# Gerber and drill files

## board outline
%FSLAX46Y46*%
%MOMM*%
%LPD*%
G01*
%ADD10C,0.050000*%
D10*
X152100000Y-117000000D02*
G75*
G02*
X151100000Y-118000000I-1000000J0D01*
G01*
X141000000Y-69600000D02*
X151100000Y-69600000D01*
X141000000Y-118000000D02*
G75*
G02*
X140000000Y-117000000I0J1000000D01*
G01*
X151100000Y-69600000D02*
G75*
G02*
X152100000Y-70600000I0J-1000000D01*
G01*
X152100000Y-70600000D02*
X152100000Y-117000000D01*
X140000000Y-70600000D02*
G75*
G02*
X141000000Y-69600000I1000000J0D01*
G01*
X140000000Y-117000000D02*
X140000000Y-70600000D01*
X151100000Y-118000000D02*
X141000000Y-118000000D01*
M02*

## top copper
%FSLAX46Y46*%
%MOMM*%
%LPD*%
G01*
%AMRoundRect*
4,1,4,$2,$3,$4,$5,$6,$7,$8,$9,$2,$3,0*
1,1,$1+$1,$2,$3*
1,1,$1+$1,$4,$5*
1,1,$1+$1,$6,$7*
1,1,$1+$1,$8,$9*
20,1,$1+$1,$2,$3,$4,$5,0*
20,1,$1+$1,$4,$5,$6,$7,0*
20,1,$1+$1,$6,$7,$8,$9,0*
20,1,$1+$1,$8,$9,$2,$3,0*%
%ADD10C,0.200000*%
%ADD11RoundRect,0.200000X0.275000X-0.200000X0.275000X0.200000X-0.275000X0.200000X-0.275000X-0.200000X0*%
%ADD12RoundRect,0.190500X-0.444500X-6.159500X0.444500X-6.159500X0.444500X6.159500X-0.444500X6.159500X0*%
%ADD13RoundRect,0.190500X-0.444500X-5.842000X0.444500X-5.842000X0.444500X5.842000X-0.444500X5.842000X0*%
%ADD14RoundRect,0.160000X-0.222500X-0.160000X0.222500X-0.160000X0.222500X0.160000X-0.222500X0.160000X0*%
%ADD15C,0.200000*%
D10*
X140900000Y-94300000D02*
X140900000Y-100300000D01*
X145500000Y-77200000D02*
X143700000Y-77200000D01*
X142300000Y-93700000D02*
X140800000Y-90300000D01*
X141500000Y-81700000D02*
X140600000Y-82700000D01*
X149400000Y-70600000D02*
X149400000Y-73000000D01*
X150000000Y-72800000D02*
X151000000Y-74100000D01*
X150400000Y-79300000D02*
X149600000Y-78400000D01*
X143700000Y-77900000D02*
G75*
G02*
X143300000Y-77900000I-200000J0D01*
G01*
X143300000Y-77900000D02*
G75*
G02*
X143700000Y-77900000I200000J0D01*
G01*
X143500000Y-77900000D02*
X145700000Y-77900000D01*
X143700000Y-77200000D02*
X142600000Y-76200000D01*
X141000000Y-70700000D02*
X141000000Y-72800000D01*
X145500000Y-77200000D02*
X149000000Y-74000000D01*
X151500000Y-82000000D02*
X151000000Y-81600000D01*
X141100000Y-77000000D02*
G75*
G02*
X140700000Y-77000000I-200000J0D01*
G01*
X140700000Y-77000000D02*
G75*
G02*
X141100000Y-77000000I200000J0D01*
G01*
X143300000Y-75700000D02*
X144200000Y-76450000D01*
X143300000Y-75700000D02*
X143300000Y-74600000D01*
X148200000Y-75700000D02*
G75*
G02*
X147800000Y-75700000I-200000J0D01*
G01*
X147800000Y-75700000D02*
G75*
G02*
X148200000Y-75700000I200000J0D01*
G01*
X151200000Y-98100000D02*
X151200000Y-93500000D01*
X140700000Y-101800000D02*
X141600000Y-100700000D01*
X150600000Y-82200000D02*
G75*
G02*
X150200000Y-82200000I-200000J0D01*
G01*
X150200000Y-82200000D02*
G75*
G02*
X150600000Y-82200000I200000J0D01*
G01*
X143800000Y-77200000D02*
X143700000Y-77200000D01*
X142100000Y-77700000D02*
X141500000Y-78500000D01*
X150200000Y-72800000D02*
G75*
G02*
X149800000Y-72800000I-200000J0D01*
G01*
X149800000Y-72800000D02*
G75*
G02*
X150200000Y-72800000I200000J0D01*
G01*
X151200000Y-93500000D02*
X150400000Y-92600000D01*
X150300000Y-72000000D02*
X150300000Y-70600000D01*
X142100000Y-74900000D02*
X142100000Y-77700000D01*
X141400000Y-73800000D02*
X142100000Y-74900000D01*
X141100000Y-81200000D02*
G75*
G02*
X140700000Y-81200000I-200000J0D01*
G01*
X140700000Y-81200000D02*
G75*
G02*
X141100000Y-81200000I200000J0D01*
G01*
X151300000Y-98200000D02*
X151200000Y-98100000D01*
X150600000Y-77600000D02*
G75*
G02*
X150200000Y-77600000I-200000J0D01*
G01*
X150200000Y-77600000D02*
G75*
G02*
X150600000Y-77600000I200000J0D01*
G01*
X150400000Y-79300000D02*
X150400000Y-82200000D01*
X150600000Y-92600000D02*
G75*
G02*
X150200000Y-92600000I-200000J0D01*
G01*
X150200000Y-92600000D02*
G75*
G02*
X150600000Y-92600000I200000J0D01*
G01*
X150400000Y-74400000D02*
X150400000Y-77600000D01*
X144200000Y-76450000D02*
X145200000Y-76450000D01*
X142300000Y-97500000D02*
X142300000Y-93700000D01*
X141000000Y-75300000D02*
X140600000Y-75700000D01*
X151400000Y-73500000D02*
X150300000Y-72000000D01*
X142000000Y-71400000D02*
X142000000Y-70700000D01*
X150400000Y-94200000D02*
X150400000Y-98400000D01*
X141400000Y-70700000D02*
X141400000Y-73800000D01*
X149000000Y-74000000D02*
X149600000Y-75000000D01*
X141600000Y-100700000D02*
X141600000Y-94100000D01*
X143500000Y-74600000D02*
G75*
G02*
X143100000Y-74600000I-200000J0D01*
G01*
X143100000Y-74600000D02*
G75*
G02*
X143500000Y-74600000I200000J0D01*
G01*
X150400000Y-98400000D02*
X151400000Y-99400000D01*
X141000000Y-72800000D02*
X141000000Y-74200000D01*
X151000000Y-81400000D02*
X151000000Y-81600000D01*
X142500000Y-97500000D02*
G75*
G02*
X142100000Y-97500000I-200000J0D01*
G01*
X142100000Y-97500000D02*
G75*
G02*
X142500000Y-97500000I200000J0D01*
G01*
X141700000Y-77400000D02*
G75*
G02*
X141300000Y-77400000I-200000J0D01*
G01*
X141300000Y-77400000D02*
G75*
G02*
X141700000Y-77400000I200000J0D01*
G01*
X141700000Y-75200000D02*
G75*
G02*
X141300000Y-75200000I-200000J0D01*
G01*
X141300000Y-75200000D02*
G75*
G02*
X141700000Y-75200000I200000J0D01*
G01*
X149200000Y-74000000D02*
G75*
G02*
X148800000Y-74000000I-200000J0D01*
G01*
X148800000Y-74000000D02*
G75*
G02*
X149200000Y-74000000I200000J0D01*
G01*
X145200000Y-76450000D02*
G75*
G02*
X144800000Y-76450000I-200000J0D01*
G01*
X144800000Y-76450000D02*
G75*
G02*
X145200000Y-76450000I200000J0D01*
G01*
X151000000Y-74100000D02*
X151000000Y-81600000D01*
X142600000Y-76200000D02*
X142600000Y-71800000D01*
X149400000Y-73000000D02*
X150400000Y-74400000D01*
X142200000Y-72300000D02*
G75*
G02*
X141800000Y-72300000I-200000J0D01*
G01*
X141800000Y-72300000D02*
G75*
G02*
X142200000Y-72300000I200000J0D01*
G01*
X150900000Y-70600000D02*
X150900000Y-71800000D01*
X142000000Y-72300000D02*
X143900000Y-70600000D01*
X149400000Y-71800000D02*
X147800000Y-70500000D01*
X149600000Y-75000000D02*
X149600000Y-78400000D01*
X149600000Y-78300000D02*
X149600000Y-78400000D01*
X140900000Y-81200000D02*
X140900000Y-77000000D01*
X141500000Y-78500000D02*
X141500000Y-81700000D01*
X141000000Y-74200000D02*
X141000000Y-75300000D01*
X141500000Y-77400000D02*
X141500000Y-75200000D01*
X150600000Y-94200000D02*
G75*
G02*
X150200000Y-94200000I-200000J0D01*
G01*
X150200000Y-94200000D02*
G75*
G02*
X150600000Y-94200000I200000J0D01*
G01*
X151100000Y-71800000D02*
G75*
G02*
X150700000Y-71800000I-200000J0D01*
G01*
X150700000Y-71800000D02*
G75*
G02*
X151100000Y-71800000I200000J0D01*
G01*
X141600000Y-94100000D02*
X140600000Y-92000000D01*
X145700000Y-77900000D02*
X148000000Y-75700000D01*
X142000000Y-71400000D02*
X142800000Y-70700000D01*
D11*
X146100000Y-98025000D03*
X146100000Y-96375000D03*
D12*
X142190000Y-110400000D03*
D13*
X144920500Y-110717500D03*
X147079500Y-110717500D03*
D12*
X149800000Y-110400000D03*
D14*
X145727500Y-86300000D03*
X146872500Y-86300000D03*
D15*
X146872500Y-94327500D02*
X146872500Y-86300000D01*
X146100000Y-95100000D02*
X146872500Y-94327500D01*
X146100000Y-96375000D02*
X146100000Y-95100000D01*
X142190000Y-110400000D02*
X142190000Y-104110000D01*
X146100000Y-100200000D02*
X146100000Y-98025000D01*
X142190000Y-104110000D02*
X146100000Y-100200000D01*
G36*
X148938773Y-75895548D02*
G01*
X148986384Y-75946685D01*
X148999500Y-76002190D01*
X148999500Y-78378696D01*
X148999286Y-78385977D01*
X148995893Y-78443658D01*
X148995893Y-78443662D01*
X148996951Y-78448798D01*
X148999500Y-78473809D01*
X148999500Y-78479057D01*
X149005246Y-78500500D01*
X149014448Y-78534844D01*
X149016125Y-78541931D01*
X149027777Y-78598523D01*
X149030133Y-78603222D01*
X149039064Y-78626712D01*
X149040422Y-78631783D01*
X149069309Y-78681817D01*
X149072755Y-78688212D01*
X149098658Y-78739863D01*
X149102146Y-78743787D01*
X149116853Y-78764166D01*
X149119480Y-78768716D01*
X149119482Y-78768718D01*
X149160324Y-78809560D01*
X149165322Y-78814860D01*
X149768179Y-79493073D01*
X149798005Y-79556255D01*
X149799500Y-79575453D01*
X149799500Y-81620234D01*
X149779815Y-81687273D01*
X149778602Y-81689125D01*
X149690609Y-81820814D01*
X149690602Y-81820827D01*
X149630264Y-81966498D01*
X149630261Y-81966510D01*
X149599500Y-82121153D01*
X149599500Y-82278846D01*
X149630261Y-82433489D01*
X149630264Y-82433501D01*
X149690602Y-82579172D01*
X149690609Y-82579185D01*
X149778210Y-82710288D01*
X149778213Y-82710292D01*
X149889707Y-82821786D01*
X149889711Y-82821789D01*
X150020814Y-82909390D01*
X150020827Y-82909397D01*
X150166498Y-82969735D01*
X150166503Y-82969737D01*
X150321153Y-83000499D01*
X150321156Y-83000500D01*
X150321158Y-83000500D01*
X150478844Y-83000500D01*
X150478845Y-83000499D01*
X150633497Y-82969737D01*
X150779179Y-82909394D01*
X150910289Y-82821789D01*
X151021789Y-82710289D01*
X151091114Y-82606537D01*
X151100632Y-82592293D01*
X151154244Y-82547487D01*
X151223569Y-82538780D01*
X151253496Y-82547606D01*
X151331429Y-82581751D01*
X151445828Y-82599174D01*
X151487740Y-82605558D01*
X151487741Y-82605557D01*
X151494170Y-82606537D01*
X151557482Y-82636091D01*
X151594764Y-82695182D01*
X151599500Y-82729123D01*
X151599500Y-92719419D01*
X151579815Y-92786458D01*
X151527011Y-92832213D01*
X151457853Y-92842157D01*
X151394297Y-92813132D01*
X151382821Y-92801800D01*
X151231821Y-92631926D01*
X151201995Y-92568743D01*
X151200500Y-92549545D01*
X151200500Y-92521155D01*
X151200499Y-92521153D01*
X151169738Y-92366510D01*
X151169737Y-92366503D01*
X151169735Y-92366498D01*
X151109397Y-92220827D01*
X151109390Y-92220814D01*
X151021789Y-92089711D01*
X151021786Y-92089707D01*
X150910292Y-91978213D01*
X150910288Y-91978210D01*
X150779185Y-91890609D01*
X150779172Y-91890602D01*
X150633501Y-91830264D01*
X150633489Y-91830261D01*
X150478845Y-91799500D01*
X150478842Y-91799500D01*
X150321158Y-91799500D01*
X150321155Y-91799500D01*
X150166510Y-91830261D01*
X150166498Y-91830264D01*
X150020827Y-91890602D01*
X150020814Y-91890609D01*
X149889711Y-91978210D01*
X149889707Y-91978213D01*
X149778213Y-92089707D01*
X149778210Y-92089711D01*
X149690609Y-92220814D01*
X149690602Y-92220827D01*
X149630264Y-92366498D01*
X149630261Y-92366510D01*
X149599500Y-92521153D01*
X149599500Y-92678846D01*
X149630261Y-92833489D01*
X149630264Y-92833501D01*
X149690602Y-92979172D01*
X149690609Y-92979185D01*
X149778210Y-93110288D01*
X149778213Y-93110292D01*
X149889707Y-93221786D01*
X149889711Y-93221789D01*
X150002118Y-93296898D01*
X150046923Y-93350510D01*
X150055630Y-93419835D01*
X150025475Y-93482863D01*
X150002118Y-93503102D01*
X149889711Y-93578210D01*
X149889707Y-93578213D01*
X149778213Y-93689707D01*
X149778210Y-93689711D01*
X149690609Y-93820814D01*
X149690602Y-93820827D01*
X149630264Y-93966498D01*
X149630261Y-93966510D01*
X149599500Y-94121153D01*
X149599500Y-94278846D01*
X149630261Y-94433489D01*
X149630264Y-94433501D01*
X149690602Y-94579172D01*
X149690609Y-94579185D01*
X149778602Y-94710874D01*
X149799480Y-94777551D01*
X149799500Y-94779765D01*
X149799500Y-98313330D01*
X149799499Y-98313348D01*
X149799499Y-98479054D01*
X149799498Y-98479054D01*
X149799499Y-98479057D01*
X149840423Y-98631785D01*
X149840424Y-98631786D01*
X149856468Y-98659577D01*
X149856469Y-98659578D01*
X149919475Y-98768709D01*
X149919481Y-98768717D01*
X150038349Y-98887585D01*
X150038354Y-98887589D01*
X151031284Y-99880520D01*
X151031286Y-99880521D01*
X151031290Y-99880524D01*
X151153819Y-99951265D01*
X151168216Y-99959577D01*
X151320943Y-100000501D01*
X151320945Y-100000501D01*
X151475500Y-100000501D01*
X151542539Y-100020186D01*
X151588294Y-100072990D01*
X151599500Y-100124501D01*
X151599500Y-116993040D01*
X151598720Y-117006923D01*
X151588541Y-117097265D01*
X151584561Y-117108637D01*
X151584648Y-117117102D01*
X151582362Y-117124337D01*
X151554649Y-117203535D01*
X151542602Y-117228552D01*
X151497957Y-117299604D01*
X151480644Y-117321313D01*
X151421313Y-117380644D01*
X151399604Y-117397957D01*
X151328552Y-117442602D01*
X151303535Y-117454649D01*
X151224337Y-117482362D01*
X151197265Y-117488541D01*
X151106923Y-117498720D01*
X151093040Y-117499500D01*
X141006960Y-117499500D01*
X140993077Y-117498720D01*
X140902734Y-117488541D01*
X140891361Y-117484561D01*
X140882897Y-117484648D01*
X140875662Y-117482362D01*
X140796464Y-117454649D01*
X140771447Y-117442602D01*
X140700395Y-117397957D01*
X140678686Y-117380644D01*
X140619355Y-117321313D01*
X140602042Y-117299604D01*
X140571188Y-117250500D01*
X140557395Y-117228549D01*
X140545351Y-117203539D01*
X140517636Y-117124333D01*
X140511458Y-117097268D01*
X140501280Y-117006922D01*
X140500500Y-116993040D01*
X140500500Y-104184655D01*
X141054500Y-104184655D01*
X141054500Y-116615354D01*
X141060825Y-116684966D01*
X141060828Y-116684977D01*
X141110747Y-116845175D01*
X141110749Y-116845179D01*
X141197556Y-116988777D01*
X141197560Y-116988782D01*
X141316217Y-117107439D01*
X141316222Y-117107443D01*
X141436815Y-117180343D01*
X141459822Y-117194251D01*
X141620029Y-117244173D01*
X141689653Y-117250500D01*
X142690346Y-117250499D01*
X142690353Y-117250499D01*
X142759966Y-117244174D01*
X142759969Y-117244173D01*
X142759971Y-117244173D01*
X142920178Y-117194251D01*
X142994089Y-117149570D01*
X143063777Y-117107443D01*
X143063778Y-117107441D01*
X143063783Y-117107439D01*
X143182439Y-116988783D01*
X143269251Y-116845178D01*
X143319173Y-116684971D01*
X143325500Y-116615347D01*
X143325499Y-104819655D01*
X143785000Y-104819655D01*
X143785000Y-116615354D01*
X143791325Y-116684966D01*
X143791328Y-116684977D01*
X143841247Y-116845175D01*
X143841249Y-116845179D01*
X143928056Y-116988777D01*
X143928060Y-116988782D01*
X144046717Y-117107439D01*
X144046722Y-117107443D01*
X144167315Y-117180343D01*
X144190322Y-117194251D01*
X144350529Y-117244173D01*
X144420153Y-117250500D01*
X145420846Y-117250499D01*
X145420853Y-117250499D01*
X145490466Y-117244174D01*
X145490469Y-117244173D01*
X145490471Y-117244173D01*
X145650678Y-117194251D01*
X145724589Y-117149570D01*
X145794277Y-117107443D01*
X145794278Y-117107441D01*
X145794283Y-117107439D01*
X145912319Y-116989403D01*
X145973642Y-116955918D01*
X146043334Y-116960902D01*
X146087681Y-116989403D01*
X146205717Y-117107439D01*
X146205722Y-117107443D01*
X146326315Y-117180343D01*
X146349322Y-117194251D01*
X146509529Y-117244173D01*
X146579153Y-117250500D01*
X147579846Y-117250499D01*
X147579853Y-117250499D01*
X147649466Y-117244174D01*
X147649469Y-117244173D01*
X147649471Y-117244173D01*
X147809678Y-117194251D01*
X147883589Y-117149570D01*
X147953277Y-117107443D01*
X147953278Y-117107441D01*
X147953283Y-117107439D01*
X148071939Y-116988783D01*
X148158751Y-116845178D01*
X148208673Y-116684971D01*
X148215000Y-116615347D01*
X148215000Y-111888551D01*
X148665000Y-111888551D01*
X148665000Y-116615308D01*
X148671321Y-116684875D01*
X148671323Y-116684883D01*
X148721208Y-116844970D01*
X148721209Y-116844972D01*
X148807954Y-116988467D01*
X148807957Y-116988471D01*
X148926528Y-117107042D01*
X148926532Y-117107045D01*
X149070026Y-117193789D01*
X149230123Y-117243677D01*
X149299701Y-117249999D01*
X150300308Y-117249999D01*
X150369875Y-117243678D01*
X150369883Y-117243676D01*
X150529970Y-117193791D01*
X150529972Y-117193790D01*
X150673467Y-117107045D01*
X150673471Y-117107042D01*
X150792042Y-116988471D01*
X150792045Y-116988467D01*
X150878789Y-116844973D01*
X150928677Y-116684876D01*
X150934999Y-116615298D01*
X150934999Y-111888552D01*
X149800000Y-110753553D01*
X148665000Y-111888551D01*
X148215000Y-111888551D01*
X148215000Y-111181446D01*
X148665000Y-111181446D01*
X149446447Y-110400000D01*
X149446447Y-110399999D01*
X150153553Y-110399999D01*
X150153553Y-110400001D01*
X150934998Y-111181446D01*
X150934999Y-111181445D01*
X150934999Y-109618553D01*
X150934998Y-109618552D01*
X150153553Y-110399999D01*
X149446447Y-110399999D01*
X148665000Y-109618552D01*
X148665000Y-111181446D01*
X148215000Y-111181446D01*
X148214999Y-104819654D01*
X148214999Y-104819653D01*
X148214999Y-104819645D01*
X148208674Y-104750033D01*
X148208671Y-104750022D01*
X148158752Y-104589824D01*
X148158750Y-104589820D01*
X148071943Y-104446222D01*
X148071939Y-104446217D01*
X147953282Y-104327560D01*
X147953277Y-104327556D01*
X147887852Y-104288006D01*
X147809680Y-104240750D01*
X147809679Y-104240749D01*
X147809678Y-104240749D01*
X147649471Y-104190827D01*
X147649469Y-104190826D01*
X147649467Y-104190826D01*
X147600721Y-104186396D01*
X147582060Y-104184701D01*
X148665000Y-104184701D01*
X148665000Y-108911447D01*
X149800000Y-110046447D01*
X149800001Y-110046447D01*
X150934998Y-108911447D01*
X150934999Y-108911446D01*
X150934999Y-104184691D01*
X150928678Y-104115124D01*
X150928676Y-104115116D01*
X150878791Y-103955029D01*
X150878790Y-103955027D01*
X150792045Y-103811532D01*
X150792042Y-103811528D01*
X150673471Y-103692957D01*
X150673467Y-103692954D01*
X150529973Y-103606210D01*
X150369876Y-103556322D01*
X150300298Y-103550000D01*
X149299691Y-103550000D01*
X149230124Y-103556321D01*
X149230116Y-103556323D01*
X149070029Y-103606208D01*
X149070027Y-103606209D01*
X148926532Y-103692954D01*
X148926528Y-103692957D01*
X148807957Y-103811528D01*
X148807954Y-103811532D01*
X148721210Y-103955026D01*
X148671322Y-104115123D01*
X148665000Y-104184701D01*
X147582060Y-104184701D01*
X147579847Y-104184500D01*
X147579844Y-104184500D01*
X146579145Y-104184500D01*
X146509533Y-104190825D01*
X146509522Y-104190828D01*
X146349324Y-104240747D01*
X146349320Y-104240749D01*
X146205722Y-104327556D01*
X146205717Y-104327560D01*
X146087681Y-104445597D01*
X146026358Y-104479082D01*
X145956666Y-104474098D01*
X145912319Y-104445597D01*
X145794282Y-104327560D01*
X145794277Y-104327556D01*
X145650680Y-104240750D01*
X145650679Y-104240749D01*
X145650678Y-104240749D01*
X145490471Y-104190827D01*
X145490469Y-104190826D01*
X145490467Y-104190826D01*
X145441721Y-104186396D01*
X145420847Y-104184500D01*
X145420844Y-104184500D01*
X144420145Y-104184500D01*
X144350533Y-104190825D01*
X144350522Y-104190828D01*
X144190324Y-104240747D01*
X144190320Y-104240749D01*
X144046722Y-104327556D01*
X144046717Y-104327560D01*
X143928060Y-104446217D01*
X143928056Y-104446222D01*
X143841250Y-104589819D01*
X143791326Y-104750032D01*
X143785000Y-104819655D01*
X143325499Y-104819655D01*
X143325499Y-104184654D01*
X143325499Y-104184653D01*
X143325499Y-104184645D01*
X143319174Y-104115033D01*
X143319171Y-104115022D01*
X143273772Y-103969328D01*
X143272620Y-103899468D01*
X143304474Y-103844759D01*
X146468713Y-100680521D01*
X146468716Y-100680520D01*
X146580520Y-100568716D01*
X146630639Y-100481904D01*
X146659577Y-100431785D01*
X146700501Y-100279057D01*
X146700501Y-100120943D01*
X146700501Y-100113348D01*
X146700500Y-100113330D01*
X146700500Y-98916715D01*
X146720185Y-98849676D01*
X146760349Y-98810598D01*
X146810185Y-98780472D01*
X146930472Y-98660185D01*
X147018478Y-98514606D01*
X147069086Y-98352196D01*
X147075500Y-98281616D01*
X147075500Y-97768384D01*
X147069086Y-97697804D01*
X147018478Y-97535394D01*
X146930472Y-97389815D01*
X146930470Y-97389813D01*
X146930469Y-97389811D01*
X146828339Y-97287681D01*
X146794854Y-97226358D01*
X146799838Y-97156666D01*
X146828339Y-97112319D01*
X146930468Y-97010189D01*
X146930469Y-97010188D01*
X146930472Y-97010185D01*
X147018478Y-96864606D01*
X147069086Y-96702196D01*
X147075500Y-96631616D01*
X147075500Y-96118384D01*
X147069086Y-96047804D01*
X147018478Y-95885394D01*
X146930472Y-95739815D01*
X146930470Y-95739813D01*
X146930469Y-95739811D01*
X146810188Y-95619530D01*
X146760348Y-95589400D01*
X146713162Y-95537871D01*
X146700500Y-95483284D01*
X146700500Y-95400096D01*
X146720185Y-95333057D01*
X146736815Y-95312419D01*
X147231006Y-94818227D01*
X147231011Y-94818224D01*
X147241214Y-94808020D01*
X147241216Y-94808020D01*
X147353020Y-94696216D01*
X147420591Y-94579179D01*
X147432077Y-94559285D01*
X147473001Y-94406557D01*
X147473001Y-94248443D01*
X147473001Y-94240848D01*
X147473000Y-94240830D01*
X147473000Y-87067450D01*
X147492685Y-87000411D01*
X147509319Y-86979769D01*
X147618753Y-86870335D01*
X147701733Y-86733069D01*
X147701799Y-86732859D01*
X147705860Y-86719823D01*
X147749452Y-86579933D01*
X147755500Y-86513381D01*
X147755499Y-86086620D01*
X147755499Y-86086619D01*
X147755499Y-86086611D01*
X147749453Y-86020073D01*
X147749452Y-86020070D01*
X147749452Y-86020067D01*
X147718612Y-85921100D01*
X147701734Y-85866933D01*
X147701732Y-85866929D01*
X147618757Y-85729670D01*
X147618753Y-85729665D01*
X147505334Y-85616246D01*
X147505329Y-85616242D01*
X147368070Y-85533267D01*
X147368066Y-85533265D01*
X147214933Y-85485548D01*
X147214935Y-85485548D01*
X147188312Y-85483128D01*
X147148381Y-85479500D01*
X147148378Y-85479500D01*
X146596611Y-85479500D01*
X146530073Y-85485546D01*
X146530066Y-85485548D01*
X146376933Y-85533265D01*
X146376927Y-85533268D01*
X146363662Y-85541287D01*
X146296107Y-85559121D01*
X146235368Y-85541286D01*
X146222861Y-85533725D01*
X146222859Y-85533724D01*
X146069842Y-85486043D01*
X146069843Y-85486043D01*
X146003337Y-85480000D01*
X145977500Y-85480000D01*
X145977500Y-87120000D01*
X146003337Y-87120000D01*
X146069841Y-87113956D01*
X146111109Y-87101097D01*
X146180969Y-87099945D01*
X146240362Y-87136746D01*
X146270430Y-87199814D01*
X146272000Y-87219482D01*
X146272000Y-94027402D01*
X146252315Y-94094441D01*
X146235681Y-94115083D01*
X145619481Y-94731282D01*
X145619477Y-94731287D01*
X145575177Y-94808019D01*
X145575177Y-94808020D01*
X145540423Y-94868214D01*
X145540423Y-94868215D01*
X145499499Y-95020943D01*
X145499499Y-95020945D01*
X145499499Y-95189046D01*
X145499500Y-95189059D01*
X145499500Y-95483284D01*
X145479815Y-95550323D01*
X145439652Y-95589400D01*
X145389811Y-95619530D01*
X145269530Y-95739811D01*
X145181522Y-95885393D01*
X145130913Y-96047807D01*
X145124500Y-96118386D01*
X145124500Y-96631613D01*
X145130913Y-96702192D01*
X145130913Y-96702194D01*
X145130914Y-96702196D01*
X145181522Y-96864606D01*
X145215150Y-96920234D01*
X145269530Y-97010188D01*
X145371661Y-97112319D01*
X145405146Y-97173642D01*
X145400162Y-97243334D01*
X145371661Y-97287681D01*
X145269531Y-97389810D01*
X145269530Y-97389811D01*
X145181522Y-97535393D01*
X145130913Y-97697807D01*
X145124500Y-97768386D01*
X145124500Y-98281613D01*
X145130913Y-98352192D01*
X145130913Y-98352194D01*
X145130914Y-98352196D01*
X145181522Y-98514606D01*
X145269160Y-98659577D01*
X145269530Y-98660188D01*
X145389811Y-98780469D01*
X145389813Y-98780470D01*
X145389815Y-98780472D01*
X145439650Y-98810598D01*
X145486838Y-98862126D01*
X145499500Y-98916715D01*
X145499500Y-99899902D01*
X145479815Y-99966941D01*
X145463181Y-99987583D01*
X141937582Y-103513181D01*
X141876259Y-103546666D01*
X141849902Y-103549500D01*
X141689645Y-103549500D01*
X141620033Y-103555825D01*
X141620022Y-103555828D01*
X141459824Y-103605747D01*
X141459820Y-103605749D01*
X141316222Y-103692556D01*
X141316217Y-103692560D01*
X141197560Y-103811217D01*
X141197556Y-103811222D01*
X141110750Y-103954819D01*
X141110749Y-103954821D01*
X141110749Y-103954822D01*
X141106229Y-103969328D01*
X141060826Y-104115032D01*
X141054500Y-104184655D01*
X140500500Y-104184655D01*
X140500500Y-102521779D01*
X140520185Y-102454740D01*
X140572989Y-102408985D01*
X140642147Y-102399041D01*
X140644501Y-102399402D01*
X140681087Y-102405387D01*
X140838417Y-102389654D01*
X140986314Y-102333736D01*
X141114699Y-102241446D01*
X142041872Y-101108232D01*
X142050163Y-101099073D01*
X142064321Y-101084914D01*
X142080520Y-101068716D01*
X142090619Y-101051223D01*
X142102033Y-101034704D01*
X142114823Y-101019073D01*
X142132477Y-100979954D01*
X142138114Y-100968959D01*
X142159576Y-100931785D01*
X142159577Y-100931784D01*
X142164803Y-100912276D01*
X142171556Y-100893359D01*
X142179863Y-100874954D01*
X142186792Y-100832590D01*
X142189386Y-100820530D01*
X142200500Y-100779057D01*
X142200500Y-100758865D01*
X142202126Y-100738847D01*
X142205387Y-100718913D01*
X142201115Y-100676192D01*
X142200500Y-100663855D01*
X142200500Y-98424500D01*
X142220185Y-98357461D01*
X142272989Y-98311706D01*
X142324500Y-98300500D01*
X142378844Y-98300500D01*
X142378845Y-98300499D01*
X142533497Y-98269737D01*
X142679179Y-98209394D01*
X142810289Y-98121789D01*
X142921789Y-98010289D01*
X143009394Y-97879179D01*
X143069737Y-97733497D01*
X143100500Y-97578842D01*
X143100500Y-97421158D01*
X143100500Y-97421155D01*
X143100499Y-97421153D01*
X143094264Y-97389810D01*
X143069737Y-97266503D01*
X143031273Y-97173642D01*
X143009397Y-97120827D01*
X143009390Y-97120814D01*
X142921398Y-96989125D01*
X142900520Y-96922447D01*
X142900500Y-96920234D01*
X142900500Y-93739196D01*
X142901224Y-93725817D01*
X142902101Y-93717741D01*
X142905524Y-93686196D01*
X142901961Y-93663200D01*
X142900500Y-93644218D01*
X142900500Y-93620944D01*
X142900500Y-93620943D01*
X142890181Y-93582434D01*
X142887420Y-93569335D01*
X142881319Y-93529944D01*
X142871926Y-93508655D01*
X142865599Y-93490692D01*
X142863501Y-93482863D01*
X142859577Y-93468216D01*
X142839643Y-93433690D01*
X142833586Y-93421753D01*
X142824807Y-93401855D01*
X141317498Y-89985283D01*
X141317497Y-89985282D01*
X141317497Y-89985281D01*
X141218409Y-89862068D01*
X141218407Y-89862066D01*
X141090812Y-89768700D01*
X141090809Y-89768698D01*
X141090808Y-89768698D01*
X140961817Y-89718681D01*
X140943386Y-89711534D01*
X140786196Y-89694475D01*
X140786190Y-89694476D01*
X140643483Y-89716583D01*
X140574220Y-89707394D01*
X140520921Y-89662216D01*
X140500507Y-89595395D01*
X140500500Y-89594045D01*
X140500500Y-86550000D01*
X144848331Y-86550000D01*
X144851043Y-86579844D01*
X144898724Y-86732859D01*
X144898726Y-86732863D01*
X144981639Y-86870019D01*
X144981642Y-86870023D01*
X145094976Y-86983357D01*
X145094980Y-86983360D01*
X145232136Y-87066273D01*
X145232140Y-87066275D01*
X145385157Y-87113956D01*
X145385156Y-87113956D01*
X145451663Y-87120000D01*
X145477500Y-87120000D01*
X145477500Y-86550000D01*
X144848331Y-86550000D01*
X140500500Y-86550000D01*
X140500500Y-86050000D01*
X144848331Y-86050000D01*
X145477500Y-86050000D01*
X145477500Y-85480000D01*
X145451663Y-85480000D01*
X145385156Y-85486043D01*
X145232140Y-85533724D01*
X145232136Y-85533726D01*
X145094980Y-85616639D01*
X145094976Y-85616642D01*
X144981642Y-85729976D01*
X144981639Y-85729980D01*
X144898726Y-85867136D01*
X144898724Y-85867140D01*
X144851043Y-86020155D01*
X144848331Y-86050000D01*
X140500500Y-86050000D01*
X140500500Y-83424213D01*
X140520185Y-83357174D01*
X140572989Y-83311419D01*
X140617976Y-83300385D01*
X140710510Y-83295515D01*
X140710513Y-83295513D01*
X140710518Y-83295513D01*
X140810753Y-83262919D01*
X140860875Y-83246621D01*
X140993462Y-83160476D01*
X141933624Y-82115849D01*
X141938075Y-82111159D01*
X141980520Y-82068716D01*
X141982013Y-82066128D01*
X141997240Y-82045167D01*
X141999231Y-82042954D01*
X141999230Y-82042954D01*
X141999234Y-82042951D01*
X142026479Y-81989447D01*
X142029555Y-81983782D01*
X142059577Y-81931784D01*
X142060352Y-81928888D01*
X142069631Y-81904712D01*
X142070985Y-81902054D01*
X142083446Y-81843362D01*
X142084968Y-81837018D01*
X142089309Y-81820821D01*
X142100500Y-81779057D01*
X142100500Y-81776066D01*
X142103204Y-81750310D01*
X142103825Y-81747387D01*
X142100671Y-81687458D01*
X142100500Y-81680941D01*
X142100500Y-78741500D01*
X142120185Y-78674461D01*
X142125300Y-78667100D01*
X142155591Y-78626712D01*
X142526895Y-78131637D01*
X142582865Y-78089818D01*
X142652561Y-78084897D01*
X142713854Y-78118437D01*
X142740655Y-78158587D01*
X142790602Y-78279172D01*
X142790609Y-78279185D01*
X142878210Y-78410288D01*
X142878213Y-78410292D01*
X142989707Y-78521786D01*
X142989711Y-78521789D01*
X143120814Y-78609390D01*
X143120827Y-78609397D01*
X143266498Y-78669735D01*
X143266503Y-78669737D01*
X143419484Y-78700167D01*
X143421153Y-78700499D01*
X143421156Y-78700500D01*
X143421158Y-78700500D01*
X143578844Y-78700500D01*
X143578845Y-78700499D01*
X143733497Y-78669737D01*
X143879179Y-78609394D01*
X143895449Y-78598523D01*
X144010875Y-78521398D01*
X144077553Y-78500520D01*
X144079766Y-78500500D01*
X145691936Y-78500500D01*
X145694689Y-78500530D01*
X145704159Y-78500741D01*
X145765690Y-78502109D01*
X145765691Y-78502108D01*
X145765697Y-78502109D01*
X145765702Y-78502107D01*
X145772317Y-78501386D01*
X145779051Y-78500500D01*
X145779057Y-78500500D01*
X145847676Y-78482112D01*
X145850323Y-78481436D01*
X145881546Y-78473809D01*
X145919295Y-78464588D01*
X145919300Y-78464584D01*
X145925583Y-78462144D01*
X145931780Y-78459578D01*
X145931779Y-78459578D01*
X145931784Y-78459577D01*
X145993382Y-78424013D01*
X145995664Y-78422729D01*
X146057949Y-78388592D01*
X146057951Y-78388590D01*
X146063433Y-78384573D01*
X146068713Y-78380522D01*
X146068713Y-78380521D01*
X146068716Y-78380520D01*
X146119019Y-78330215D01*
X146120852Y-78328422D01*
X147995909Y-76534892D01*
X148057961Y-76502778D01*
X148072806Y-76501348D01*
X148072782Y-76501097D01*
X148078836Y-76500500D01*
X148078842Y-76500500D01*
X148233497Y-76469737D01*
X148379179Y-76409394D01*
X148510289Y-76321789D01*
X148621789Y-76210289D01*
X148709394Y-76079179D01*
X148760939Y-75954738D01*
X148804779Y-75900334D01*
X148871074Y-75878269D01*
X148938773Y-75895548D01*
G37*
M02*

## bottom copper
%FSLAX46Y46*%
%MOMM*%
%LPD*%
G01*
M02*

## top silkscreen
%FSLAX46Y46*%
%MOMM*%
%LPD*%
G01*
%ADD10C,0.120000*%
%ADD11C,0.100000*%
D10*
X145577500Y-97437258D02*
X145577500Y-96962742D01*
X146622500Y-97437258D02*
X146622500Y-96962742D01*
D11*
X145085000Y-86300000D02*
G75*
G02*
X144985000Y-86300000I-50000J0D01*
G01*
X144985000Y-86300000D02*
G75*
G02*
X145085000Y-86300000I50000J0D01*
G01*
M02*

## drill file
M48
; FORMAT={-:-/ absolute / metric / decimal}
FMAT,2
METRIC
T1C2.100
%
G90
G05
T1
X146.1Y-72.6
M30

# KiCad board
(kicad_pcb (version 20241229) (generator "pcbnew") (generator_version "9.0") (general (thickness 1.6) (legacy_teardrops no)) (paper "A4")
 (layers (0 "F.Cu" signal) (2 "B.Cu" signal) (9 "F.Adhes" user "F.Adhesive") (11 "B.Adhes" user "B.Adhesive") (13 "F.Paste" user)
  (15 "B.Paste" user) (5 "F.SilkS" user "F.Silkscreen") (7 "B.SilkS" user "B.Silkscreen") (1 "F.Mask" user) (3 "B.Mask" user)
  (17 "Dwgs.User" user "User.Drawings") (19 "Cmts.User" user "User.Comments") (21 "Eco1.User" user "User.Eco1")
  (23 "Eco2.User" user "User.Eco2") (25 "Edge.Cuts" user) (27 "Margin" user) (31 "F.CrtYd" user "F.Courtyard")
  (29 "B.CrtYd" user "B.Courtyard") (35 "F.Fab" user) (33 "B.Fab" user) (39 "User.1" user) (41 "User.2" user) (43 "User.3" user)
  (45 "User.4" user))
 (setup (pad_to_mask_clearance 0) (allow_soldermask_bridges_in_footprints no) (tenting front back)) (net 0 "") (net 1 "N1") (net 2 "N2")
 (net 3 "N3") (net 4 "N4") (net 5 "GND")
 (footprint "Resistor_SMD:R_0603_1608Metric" (layer "F.Cu") (at 146.1 97.2 90)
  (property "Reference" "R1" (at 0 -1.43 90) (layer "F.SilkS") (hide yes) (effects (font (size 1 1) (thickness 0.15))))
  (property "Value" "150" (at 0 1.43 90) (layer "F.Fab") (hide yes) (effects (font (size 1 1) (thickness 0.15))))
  (fp_line (start -0.237258 -0.5225) (end 0.237258 -0.5225) (stroke (width 0.12) (type solid)) (layer "F.SilkS"))
  (fp_line (start -0.237258 0.5225) (end 0.237258 0.5225) (stroke (width 0.12) (type solid)) (layer "F.SilkS"))
  (pad "1" smd roundrect (at -0.825 0 90) (size 0.8 0.95) (layers "F.Cu" "F.Mask" "F.Paste") (roundrect_rratio 0.25) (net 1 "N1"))
  (pad "2" smd roundrect (at 0.825 0 90) (size 0.8 0.95) (layers "F.Cu" "F.Mask" "F.Paste") (roundrect_rratio 0.25) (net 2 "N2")))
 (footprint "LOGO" (layer "F.Cu") (at 146 81.9)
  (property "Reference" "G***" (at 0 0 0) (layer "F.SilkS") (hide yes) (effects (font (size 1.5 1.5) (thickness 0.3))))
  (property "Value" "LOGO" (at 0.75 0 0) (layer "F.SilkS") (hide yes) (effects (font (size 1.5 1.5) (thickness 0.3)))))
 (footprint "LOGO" (layer "F.Cu") (at 142.8 87.2)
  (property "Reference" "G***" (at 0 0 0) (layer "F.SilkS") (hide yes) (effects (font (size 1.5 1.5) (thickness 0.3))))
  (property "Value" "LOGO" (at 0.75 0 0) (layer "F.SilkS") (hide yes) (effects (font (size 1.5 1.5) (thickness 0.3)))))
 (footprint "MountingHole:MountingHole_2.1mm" (layer "F.Cu") (at 146.1 72.6)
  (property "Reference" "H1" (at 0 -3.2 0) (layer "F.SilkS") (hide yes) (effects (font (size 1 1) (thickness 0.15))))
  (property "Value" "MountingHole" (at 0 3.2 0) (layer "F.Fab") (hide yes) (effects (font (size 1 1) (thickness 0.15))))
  (pad "" np_thru_hole circle (at 0 0) (size 2.1 2.1) (drill 2.1) (layers "*.Cu" "*.Mask")))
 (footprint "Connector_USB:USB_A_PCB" (layer "F.Cu") (at 146 110.0825)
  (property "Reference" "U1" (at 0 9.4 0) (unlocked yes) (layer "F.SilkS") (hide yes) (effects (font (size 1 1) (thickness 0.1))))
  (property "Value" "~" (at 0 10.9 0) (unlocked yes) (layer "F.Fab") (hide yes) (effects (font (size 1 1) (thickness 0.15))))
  (pad "1" smd roundrect (at -3.81 0.3175) (size 1.27 12.7) (layers "F.Cu" "F.Mask" "F.Paste") (roundrect_rratio 0.15) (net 1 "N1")
   (thermal_bridge_angle 45))
  (pad "2" smd roundrect (at -1.0795 0.635) (size 1.27 12.065) (layers "F.Cu" "F.Mask" "F.Paste") (roundrect_rratio 0.15) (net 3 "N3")
   (thermal_bridge_angle 45))
  (pad "3" smd roundrect (at 1.0795 0.635) (size 1.27 12.065) (layers "F.Cu" "F.Mask" "F.Paste") (roundrect_rratio 0.15) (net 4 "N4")
   (thermal_bridge_angle 45))
  (pad "4" smd roundrect (at 3.8 0.3175) (size 1.27 12.7) (layers "F.Cu" "F.Mask" "F.Paste") (roundrect_rratio 0.15) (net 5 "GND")
   (thermal_bridge_angle 45)))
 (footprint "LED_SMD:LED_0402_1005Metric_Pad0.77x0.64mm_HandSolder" (layer "F.Cu") (at 146.3 86.3)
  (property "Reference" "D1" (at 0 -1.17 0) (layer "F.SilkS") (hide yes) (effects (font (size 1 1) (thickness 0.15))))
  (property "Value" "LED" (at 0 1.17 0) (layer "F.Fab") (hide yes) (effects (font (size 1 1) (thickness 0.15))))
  (fp_circle (center -1.265 0) (end -1.215 0) (stroke (width 0.1) (type solid)) (fill no) (layer "F.SilkS"))
  (pad "1" smd roundrect (at -0.5725 0) (size 0.765 0.64) (layers "F.Cu" "F.Mask" "F.Paste") (roundrect_rratio 0.25) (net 5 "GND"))
  (pad "2" smd roundrect (at 0.5725 0) (size 0.765 0.64) (layers "F.Cu" "F.Mask" "F.Paste") (roundrect_rratio 0.25) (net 2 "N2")))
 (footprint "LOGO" (layer "F.Cu") (at 149.7 87.2)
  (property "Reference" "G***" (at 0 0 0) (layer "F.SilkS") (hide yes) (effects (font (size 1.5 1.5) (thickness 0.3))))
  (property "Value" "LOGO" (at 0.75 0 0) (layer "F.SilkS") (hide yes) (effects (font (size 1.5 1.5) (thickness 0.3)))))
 (gr_line (start 140.9 94.3) (end 140.9 100.3) (stroke (width 0.2) (type default)) (layer "F.Cu"))
 (gr_line (start 145.5 77.2) (end 143.7 77.2) (stroke (width 0.2) (type default)) (layer "F.Cu"))
 (gr_line (start 142.3 93.7) (end 140.8 90.3) (stroke (width 0.2) (type default)) (layer "F.Cu"))
 (gr_line (start 141.5 81.7) (end 140.6 82.7) (stroke (width 0.2) (type default)) (layer "F.Cu"))
 (gr_line (start 149.4 70.6) (end 149.4 73) (stroke (width 0.2) (type default)) (layer "F.Cu"))
 (gr_line (start 150 72.8) (end 151 74.1) (stroke (width 0.2) (type default)) (layer "F.Cu"))
 (gr_line (start 150.4 79.3) (end 149.6 78.4) (stroke (width 0.2) (type default)) (layer "F.Cu"))
 (gr_circle (center 143.5 77.9) (end 143.7 77.9) (stroke (width 0.2) (type solid)) (fill no) (layer "F.Cu"))
 (gr_line (start 143.5 77.9) (end 145.7 77.9) (stroke (width 0.2) (type default)) (layer "F.Cu"))
 (gr_line (start 143.7 77.2) (end 142.6 76.2) (stroke (width 0.2) (type default)) (layer "F.Cu"))
 (gr_line (start 141 70.7) (end 141 72.8) (stroke (width 0.2) (type default)) (layer "F.Cu"))
 (gr_line (start 145.5 77.2) (end 149 74) (stroke (width 0.2) (type default)) (layer "F.Cu"))
 (gr_line (start 151.5 82) (end 151 81.6) (stroke (width 0.2) (type default)) (layer "F.Cu"))
 (gr_circle (center 140.9 77) (end 141.1 77) (stroke (width 0.2) (type solid)) (fill no) (layer "F.Cu"))
 (gr_line (start 143.3 75.7) (end 144.2 76.45) (stroke (width 0.2) (type default)) (layer "F.Cu"))
 (gr_line (start 143.3 75.7) (end 143.3 74.6) (stroke (width 0.2) (type default)) (layer "F.Cu"))
 (gr_circle (center 148 75.7) (end 148.2 75.7) (stroke (width 0.2) (type solid)) (fill no) (layer "F.Cu"))
 (gr_line (start 151.2 98.1) (end 151.2 93.5) (stroke (width 0.2) (type default)) (layer "F.Cu"))
 (gr_line (start 140.7 101.8) (end 141.6 100.7) (stroke (width 0.2) (type default)) (layer "F.Cu"))
 (gr_circle (center 150.4 82.2) (end 150.6 82.2) (stroke (width 0.2) (type solid)) (fill no) (layer "F.Cu"))
 (gr_line (start 143.8 77.2) (end 143.7 77.2) (stroke (width 0.2) (type default)) (layer "F.Cu"))
 (gr_line (start 142.1 77.7) (end 141.5 78.5) (stroke (width 0.2) (type default)) (layer "F.Cu"))
 (gr_circle (center 150 72.8) (end 150.2 72.8) (stroke (width 0.2) (type solid)) (fill no) (layer "F.Cu"))
 (gr_line (start 151.2 93.5) (end 150.4 92.6) (stroke (width 0.2) (type default)) (layer "F.Cu"))
 (gr_line (start 150.3 72) (end 150.3 70.6) (stroke (width 0.2) (type default)) (layer "F.Cu"))
 (gr_line (start 142.1 74.9) (end 142.1 77.7) (stroke (width 0.2) (type default)) (layer "F.Cu"))
 (gr_line (start 141.4 73.8) (end 142.1 74.9) (stroke (width 0.2) (type default)) (layer "F.Cu"))
 (gr_circle (center 140.9 81.2) (end 141.1 81.2) (stroke (width 0.2) (type solid)) (fill no) (layer "F.Cu"))
 (gr_line (start 151.3 98.2) (end 151.2 98.1) (stroke (width 0.2) (type default)) (layer "F.Cu"))
 (gr_circle (center 150.4 77.6) (end 150.6 77.6) (stroke (width 0.2) (type solid)) (fill no) (layer "F.Cu"))
 (gr_line (start 150.4 79.3) (end 150.4 82.2) (stroke (width 0.2) (type default)) (layer "F.Cu"))
 (gr_circle (center 150.4 92.6) (end 150.6 92.6) (stroke (width 0.2) (type solid)) (fill no) (layer "F.Cu"))
 (gr_line (start 150.4 74.4) (end 150.4 77.6) (stroke (width 0.2) (type default)) (layer "F.Cu"))
 (gr_line (start 144.2 76.45) (end 145.2 76.45) (stroke (width 0.2) (type default)) (layer "F.Cu"))
 (gr_line (start 142.3 97.5) (end 142.3 93.7) (stroke (width 0.2) (type default)) (layer "F.Cu"))
 (gr_line (start 141 75.3) (end 140.6 75.7) (stroke (width 0.2) (type default)) (layer "F.Cu"))
 (gr_line (start 151.4 73.5) (end 150.3 72) (stroke (width 0.2) (type default)) (layer "F.Cu"))
 (gr_line (start 142 71.4) (end 142 70.7) (stroke (width 0.2) (type default)) (layer "F.Cu"))
 (gr_line (start 150.4 94.2) (end 150.4 98.4) (stroke (width 0.2) (type default)) (layer "F.Cu"))
 (gr_line (start 141.4 70.7) (end 141.4 73.8) (stroke (width 0.2) (type default)) (layer "F.Cu"))
 (gr_line (start 149 74) (end 149.6 75) (stroke (width 0.2) (type default)) (layer "F.Cu"))
 (gr_line (start 141.6 100.7) (end 141.6 94.1) (stroke (width 0.2) (type default)) (layer "F.Cu"))
 (gr_circle (center 143.3 74.6) (end 143.5 74.6) (stroke (width 0.2) (type solid)) (fill no) (layer "F.Cu"))
 (gr_line (start 150.4 98.4) (end 151.4 99.4) (stroke (width 0.2) (type default)) (layer "F.Cu"))
 (gr_line (start 141 72.8) (end 141 74.2) (stroke (width 0.2) (type default)) (layer "F.Cu"))
 (gr_line (start 151 81.4) (end 151 81.6) (stroke (width 0.2) (type default)) (layer "F.Cu"))
 (gr_circle (center 142.3 97.5) (end 142.5 97.5) (stroke (width 0.2) (type solid)) (fill no) (layer "F.Cu"))
 (gr_circle (center 141.5 77.4) (end 141.7 77.4) (stroke (width 0.2) (type solid)) (fill no) (layer "F.Cu"))
 (gr_circle (center 141.5 75.2) (end 141.7 75.2) (stroke (width 0.2) (type solid)) (fill no) (layer "F.Cu"))
 (gr_circle (center 149 74) (end 149.2 74) (stroke (width 0.2) (type solid)) (fill no) (layer "F.Cu"))
 (gr_circle (center 145 76.45) (end 145.2 76.45) (stroke (width 0.2) (type solid)) (fill no) (layer "F.Cu"))
 (gr_line (start 151 74.1) (end 151 81.6) (stroke (width 0.2) (type default)) (layer "F.Cu"))
 (gr_line (start 142.6 76.2) (end 142.6 71.8) (stroke (width 0.2) (type default)) (layer "F.Cu"))
 (gr_line (start 149.4 73) (end 150.4 74.4) (stroke (width 0.2) (type default)) (layer "F.Cu"))
 (gr_circle (center 142 72.3) (end 142.2 72.3) (stroke (width 0.2) (type solid)) (fill no) (layer "F.Cu"))
 (gr_line (start 150.9 70.6) (end 150.9 71.8) (stroke (width 0.2) (type default)) (layer "F.Cu"))
 (gr_line (start 142 72.3) (end 143.9 70.6) (stroke (width 0.2) (type default)) (layer "F.Cu"))
 (gr_line (start 149.4 71.8) (end 147.8 70.5) (stroke (width 0.2) (type default)) (layer "F.Cu"))
 (gr_line (start 149.6 75) (end 149.6 78.4) (stroke (width 0.2) (type default)) (layer "F.Cu"))
 (gr_line (start 149.6 78.3) (end 149.6 78.4) (stroke (width 0.2) (type default)) (layer "F.Cu"))
 (gr_line (start 140.9 81.2) (end 140.9 77) (stroke (width 0.2) (type default)) (layer "F.Cu"))
 (gr_line (start 141.5 78.5) (end 141.5 81.7) (stroke (width 0.2) (type default)) (layer "F.Cu"))
 (gr_line (start 141 74.2) (end 141 75.3) (stroke (width 0.2) (type default)) (layer "F.Cu"))
 (gr_line (start 141.5 77.4) (end 141.5 75.2) (stroke (width 0.2) (type default)) (layer "F.Cu"))
 (gr_circle (center 150.4 94.2) (end 150.6 94.2) (stroke (width 0.2) (type solid)) (fill no) (layer "F.Cu"))
 (gr_circle (center 150.9 71.8) (end 151.1 71.8) (stroke (width 0.2) (type solid)) (fill no) (layer "F.Cu"))
 (gr_line (start 141.6 94.1) (end 140.6 92) (stroke (width 0.2) (type default)) (layer "F.Cu"))
 (gr_line (start 145.7 77.9) (end 148 75.7) (stroke (width 0.2) (type default)) (layer "F.Cu"))
 (gr_line (start 142 71.4) (end 142.8 70.7) (stroke (width 0.2) (type default)) (layer "F.Cu"))
 (gr_arc (start 152.1 117) (mid 151.807107 117.707107) (end 151.1 118) (stroke (width 0.05) (type default)) (layer "Edge.Cuts"))
 (gr_line (start 141 69.6) (end 151.1 69.6) (stroke (width 0.05) (type default)) (layer "Edge.Cuts"))
 (gr_arc (start 141 118) (mid 140.292893 117.707107) (end 140 117) (stroke (width 0.05) (type default)) (layer "Edge.Cuts"))
 (gr_arc (start 151.1 69.6) (mid 151.807107 69.892893) (end 152.1 70.6) (stroke (width 0.05) (type default)) (layer "Edge.Cuts"))
 (gr_line (start 152.1 70.6) (end 152.1 117) (stroke (width 0.05) (type default)) (layer "Edge.Cuts"))
 (gr_arc (start 140 70.6) (mid 140.292893 69.892893) (end 141 69.6) (stroke (width 0.05) (type default)) (layer "Edge.Cuts"))
 (gr_line (start 140 117) (end 140 70.6) (stroke (width 0.05) (type default)) (layer "Edge.Cuts"))
 (gr_line (start 151.1 118) (end 141 118) (stroke (width 0.05) (type default)) (layer "Edge.Cuts"))
 (segment (start 146.8725 94.3275) (end 146.8725 86.3) (width 0.2) (layer "F.Cu") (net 2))
 (segment (start 146.1 95.1) (end 146.8725 94.3275) (width 0.2) (layer "F.Cu") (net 2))
 (segment (start 146.1 96.375) (end 146.1 95.1) (width 0.2) (layer "F.Cu") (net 2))
 (segment (start 142.19 110.4) (end 142.19 104.11) (width 0.2) (layer "F.Cu") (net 1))
 (segment (start 146.1 100.2) (end 146.1 98.025) (width 0.2) (layer "F.Cu") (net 1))
 (segment (start 142.19 104.11) (end 146.1 100.2) (width 0.2) (layer "F.Cu") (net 1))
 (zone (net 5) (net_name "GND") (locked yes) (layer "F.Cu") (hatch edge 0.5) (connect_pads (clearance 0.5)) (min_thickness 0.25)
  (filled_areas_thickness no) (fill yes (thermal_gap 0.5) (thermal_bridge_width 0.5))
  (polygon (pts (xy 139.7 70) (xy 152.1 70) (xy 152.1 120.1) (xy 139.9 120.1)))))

